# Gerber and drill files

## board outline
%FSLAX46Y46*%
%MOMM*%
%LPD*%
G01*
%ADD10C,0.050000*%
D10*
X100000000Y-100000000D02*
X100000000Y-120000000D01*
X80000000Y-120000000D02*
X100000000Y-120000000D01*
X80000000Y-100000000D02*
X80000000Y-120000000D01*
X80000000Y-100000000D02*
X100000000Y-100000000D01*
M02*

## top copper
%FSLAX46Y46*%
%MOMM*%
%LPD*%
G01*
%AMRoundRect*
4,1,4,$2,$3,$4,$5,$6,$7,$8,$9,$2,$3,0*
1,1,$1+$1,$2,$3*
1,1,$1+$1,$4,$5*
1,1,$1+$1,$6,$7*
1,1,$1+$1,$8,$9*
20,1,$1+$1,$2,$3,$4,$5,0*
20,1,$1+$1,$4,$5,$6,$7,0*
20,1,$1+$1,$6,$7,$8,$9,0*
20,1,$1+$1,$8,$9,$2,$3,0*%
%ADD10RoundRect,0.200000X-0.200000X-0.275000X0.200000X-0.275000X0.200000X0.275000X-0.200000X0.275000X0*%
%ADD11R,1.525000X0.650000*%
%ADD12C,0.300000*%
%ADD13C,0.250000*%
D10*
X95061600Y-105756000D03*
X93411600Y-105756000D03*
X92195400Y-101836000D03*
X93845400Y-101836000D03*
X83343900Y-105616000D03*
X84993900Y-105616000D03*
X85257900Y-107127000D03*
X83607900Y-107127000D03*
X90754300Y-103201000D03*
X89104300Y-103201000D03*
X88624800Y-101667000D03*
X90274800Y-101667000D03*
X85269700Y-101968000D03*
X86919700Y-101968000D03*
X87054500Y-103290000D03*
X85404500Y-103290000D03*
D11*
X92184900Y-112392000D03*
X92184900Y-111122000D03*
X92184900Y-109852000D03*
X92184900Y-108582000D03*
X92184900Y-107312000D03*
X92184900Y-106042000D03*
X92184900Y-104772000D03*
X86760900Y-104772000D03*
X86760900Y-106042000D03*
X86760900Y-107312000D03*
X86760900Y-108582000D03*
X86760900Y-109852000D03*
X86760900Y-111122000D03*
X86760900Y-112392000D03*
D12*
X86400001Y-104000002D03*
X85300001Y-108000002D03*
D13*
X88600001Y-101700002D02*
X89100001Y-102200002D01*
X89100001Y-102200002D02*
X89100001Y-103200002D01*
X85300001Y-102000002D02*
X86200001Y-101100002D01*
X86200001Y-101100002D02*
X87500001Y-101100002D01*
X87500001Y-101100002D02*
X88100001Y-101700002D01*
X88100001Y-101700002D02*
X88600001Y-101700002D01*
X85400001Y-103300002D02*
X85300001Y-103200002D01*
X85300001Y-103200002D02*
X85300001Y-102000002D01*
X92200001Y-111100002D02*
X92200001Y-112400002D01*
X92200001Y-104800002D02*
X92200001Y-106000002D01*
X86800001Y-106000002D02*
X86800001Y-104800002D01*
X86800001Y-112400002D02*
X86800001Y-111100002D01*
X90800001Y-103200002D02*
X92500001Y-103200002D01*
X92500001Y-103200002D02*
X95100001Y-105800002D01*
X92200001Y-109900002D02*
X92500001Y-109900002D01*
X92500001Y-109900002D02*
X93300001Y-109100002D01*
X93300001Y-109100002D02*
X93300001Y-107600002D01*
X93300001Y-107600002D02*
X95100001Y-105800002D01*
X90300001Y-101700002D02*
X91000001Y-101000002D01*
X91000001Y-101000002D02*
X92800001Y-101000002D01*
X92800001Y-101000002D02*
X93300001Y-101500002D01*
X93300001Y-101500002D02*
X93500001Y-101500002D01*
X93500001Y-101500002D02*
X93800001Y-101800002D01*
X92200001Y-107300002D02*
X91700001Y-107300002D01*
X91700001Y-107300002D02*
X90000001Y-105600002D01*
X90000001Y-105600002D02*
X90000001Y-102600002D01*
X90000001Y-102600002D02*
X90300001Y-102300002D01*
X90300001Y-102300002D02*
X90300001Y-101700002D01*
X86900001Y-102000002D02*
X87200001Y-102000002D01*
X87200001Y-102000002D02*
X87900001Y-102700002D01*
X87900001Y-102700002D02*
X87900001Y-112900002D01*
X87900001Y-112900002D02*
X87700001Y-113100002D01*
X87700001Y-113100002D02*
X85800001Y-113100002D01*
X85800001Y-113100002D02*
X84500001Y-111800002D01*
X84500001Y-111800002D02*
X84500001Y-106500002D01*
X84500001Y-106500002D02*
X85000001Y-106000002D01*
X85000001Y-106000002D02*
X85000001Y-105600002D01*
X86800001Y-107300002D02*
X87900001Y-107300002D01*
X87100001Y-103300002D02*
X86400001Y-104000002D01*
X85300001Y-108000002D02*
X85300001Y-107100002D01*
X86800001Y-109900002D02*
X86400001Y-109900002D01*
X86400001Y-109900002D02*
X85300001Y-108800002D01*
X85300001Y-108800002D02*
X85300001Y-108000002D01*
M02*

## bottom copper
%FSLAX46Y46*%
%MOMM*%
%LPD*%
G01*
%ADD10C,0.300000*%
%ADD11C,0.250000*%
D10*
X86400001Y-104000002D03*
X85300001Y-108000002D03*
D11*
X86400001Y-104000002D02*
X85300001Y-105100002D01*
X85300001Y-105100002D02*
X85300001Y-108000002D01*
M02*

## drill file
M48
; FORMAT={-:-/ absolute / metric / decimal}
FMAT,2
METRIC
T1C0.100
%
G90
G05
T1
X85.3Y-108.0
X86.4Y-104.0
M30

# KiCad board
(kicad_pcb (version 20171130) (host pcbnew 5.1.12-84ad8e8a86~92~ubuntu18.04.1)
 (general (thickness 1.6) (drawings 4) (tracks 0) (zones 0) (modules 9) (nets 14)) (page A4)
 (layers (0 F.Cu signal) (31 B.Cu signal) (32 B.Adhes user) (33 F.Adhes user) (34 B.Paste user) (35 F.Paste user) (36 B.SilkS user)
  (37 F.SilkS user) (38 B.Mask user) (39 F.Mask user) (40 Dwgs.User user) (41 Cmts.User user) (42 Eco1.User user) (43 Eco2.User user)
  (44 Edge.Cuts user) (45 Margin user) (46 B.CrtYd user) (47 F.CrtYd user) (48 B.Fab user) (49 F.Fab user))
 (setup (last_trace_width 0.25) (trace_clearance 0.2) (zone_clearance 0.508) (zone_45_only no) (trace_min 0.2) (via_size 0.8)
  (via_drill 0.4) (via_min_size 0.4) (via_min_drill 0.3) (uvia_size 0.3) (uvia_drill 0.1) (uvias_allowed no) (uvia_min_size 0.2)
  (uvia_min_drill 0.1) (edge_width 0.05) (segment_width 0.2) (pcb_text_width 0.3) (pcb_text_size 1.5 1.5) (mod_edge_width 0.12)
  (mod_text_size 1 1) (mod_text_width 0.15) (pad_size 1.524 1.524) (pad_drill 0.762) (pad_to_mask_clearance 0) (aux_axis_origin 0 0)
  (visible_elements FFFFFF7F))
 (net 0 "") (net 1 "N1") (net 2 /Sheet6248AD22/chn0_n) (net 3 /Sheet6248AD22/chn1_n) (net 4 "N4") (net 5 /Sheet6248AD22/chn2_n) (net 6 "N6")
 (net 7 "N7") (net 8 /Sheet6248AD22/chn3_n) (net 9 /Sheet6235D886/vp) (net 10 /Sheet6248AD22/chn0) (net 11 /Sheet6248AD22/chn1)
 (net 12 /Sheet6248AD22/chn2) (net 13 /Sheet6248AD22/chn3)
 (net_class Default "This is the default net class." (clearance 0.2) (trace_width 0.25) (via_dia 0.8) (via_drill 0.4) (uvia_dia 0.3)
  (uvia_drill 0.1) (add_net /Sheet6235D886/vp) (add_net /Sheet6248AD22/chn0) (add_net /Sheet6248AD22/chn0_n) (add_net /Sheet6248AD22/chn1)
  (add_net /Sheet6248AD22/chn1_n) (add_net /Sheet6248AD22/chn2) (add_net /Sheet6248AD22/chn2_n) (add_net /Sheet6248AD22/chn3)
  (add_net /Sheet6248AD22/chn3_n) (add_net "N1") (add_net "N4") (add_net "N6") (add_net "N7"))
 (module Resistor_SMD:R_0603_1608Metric (layer F.Cu) (at 94.236600 105.756000)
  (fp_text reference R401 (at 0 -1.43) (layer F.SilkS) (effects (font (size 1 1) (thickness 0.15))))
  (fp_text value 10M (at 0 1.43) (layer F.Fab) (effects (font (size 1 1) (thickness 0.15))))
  (pad 2 smd roundrect (at 0.825 0) (size 0.8 0.95) (layers F.Cu F.Mask F.Paste) (roundrect_rratio 0.25) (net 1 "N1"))
  (pad 1 smd roundrect (at -0.825 0) (size 0.8 0.95) (layers F.Cu F.Mask F.Paste) (roundrect_rratio 0.25) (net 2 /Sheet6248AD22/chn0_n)))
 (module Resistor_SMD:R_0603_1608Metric (layer F.Cu) (at 93.020400 101.836000)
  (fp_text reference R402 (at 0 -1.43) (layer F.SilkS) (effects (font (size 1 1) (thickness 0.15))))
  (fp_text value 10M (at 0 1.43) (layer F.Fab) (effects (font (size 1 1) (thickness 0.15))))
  (pad 1 smd roundrect (at -0.825 0) (size 0.8 0.95) (layers F.Cu F.Mask F.Paste) (roundrect_rratio 0.25) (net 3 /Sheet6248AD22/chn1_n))
  (pad 2 smd roundrect (at 0.825 0) (size 0.8 0.95) (layers F.Cu F.Mask F.Paste) (roundrect_rratio 0.25) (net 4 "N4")))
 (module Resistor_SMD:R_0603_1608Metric (layer F.Cu) (at 84.168900 105.616000)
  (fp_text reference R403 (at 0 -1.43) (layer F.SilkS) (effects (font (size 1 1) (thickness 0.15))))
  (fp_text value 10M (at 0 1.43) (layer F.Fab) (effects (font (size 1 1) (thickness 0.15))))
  (pad 1 smd roundrect (at -0.825 0) (size 0.8 0.95) (layers F.Cu F.Mask F.Paste) (roundrect_rratio 0.25) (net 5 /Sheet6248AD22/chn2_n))
  (pad 2 smd roundrect (at 0.825 0) (size 0.8 0.95) (layers F.Cu F.Mask F.Paste) (roundrect_rratio 0.25) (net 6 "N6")))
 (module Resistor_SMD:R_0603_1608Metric (layer F.Cu) (at 84.432900 107.127000)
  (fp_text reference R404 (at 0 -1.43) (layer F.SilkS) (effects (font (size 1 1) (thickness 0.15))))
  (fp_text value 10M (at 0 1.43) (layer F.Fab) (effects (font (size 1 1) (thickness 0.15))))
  (pad 2 smd roundrect (at 0.825 0) (size 0.8 0.95) (layers F.Cu F.Mask F.Paste) (roundrect_rratio 0.25) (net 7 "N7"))
  (pad 1 smd roundrect (at -0.825 0) (size 0.8 0.95) (layers F.Cu F.Mask F.Paste) (roundrect_rratio 0.25) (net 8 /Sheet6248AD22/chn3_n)))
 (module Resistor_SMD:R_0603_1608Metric (layer F.Cu) (at 89.929300 103.201000)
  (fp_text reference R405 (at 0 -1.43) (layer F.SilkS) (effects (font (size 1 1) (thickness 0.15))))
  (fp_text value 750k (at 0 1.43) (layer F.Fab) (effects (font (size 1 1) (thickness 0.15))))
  (pad 2 smd roundrect (at 0.825 0) (size 0.8 0.95) (layers F.Cu F.Mask F.Paste) (roundrect_rratio 0.25) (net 1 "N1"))
  (pad 1 smd roundrect (at -0.825 0) (size 0.8 0.95) (layers F.Cu F.Mask F.Paste) (roundrect_rratio 0.25) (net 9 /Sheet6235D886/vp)))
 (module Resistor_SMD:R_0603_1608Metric (layer F.Cu) (at 89.449800 101.667000)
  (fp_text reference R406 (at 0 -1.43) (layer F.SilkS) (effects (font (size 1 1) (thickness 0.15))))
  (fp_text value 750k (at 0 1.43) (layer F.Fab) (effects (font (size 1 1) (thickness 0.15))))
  (pad 1 smd roundrect (at -0.825 0) (size 0.8 0.95) (layers F.Cu F.Mask F.Paste) (roundrect_rratio 0.25) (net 9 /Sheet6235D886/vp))
  (pad 2 smd roundrect (at 0.825 0) (size 0.8 0.95) (layers F.Cu F.Mask F.Paste) (roundrect_rratio 0.25) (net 4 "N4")))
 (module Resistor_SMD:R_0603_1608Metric (layer F.Cu) (at 86.094700 101.968000)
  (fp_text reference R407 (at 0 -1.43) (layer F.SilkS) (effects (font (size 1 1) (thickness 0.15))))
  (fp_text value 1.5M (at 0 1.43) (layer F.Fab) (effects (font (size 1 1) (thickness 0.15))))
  (pad 1 smd roundrect (at -0.825 0) (size 0.8 0.95) (layers F.Cu F.Mask F.Paste) (roundrect_rratio 0.25) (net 9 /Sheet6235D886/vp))
  (pad 2 smd roundrect (at 0.825 0) (size 0.8 0.95) (layers F.Cu F.Mask F.Paste) (roundrect_rratio 0.25) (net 6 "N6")))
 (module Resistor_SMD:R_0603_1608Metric (layer F.Cu) (at 86.229500 103.290000)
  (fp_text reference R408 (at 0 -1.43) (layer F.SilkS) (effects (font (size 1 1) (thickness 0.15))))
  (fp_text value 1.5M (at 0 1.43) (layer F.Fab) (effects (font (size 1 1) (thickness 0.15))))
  (pad 2 smd roundrect (at 0.825 0) (size 0.8 0.95) (layers F.Cu F.Mask F.Paste) (roundrect_rratio 0.25) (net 7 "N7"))
  (pad 1 smd roundrect (at -0.825 0) (size 0.8 0.95) (layers F.Cu F.Mask F.Paste) (roundrect_rratio 0.25) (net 9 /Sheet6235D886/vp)))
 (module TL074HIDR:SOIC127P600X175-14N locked (layer F.Cu) (at 89.472900 108.582000 180.000000)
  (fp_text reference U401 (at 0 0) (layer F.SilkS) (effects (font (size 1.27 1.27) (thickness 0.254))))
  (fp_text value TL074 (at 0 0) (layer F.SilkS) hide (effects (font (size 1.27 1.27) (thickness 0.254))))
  (pad 1 smd rect (at -2.712 -3.81 270.000000) (size 0.65 1.525) (layers F.Cu F.Mask F.Paste) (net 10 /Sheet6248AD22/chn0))
  (pad 2 smd rect (at -2.712 -2.54 270.000000) (size 0.65 1.525) (layers F.Cu F.Mask F.Paste) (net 10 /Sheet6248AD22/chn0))
  (pad 3 smd rect (at -2.712 -1.27 270.000000) (size 0.65 1.525) (layers F.Cu F.Mask F.Paste) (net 1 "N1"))
  (pad 4 smd rect (at -2.712 0 270.000000) (size 0.65 1.525) (layers F.Cu F.Mask F.Paste))
  (pad 5 smd rect (at -2.712 1.27 270.000000) (size 0.65 1.525) (layers F.Cu F.Mask F.Paste) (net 4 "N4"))
  (pad 6 smd rect (at -2.712 2.54 270.000000) (size 0.65 1.525) (layers F.Cu F.Mask F.Paste) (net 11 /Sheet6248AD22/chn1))
  (pad 7 smd rect (at -2.712 3.81 270.000000) (size 0.65 1.525) (layers F.Cu F.Mask F.Paste) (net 11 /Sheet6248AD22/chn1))
  (pad 8 smd rect (at 2.712 3.81 270.000000) (size 0.65 1.525) (layers F.Cu F.Mask F.Paste) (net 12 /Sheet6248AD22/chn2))
  (pad 9 smd rect (at 2.712 2.54 270.000000) (size 0.65 1.525) (layers F.Cu F.Mask F.Paste) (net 12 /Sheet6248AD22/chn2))
  (pad 10 smd rect (at 2.712 1.27 270.000000) (size 0.65 1.525) (layers F.Cu F.Mask F.Paste) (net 6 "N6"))
  (pad 11 smd rect (at 2.712 0 270.000000) (size 0.65 1.525) (layers F.Cu F.Mask F.Paste))
  (pad 12 smd rect (at 2.712 -1.27 270.000000) (size 0.65 1.525) (layers F.Cu F.Mask F.Paste) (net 7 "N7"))
  (pad 13 smd rect (at 2.712 -2.54 270.000000) (size 0.65 1.525) (layers F.Cu F.Mask F.Paste) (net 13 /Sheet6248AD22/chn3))
  (pad 14 smd rect (at 2.712 -3.81 270.000000) (size 0.65 1.525) (layers F.Cu F.Mask F.Paste) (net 13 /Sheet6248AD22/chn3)))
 (gr_line (start 100 100) (end 100 120) (layer Edge.Cuts) (width 0.05))
 (gr_line (start 80 120) (end 100 120) (layer Edge.Cuts) (width 0.05))
 (gr_line (start 80 100) (end 80 120) (layer Edge.Cuts) (width 0.05))
 (gr_line (start 80 100) (end 100 100) (layer Edge.Cuts) (width 0.05))
 (segment (start 88.600001 101.700002) (end 89.100001 102.200002) (width 0.250000) (layer F.Cu) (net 9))
 (segment (start 89.100001 102.200002) (end 89.100001 103.200002) (width 0.250000) (layer F.Cu) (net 9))
 (segment (start 85.300001 102.000002) (end 86.200001 101.100002) (width 0.250000) (layer F.Cu) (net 9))
 (segment (start 86.200001 101.100002) (end 87.500001 101.100002) (width 0.250000) (layer F.Cu) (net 9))
 (segment (start 87.500001 101.100002) (end 88.100001 101.700002) (width 0.250000) (layer F.Cu) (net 9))
 (segment (start 88.100001 101.700002) (end 88.600001 101.700002) (width 0.250000) (layer F.Cu) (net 9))
 (segment (start 85.400001 103.300002) (end 85.300001 103.200002) (width 0.250000) (layer F.Cu) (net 9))
 (segment (start 85.300001 103.200002) (end 85.300001 102.000002) (width 0.250000) (layer F.Cu) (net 9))
 (segment (start 92.200001 111.100002) (end 92.200001 112.400002) (width 0.250000) (layer F.Cu) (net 10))
 (segment (start 92.200001 104.800002) (end 92.200001 106.000002) (width 0.250000) (layer F.Cu) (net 11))
 (segment (start 86.800001 106.000002) (end 86.800001 104.800002) (width 0.250000) (layer F.Cu) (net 12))
 (segment (start 86.800001 112.400002) (end 86.800001 111.100002) (width 0.250000) (layer F.Cu) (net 13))
 (segment (start 90.800001 103.200002) (end 92.500001 103.200002) (width 0.250000) (layer F.Cu) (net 1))
 (segment (start 92.500001 103.200002) (end 95.100001 105.800002) (width 0.250000) (layer F.Cu) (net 1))
 (segment (start 92.200001 109.900002) (end 92.500001 109.900002) (width 0.250000) (layer F.Cu) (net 1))
 (segment (start 92.500001 109.900002) (end 93.300001 109.100002) (width 0.250000) (layer F.Cu) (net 1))
 (segment (start 93.300001 109.100002) (end 93.300001 107.600002) (width 0.250000) (layer F.Cu) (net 1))
 (segment (start 93.300001 107.600002) (end 95.100001 105.800002) (width 0.250000) (layer F.Cu) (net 1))
 (segment (start 90.300001 101.700002) (end 91.000001 101.000002) (width 0.250000) (layer F.Cu) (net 4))
 (segment (start 91.000001 101.000002) (end 92.800001 101.000002) (width 0.250000) (layer F.Cu) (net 4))
 (segment (start 92.800001 101.000002) (end 93.300001 101.500002) (width 0.250000) (layer F.Cu) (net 4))
 (segment (start 93.300001 101.500002) (end 93.500001 101.500002) (width 0.250000) (layer F.Cu) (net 4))
 (segment (start 93.500001 101.500002) (end 93.800001 101.800002) (width 0.250000) (layer F.Cu) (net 4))
 (segment (start 92.200001 107.300002) (end 91.700001 107.300002) (width 0.250000) (layer F.Cu) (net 4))
 (segment (start 91.700001 107.300002) (end 90.000001 105.600002) (width 0.250000) (layer F.Cu) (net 4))
 (segment (start 90.000001 105.600002) (end 90.000001 102.600002) (width 0.250000) (layer F.Cu) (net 4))
 (segment (start 90.000001 102.600002) (end 90.300001 102.300002) (width 0.250000) (layer F.Cu) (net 4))
 (segment (start 90.300001 102.300002) (end 90.300001 101.700002) (width 0.250000) (layer F.Cu) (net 4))
 (segment (start 86.900001 102.000002) (end 87.200001 102.000002) (width 0.250000) (layer F.Cu) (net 6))
 (segment (start 87.200001 102.000002) (end 87.900001 102.700002) (width 0.250000) (layer F.Cu) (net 6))
 (segment (start 87.900001 102.700002) (end 87.900001 112.900002) (width 0.250000) (layer F.Cu) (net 6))
 (segment (start 87.900001 112.900002) (end 87.700001 113.100002) (width 0.250000) (layer F.Cu) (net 6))
 (segment (start 87.700001 113.100002) (end 85.800001 113.100002) (width 0.250000) (layer F.Cu) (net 6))
 (segment (start 85.800001 113.100002) (end 84.500001 111.800002) (width 0.250000) (layer F.Cu) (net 6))
 (segment (start 84.500001 111.800002) (end 84.500001 106.500002) (width 0.250000) (layer F.Cu) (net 6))
 (segment (start 84.500001 106.500002) (end 85.000001 106.000002) (width 0.250000) (layer F.Cu) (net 6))
 (segment (start 85.000001 106.000002) (end 85.000001 105.600002) (width 0.250000) (layer F.Cu) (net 6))
 (segment (start 86.800001 107.300002) (end 87.900001 107.300002) (width 0.250000) (layer F.Cu) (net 6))
 (segment (start 87.100001 103.300002) (end 86.400001 104.000002) (width 0.250000) (layer F.Cu) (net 7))
 (segment (start 86.400001 104.000002) (end 85.300001 105.100002) (width 0.250000) (layer B.Cu) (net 7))
 (segment (start 85.300001 105.100002) (end 85.300001 108.000002) (width 0.250000) (layer B.Cu) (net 7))
 (segment (start 85.300001 108.000002) (end 85.300001 107.100002) (width 0.250000) (layer F.Cu) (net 7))
 (segment (start 86.800001 109.900002) (end 86.400001 109.900002) (width 0.250000) (layer F.Cu) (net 7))
 (segment (start 86.400001 109.900002) (end 85.300001 108.800002) (width 0.250000) (layer F.Cu) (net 7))
 (segment (start 85.300001 108.800002) (end 85.300001 108.000002) (width 0.250000) (layer F.Cu) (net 7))
 (via micro (at 86.400001 104.000002) (size 0.300000) (drill 0.100000) (layers F.Cu B.Cu) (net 7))
 (via micro (at 85.300001 108.000002) (size 0.300000) (drill 0.100000) (layers F.Cu B.Cu) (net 7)))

